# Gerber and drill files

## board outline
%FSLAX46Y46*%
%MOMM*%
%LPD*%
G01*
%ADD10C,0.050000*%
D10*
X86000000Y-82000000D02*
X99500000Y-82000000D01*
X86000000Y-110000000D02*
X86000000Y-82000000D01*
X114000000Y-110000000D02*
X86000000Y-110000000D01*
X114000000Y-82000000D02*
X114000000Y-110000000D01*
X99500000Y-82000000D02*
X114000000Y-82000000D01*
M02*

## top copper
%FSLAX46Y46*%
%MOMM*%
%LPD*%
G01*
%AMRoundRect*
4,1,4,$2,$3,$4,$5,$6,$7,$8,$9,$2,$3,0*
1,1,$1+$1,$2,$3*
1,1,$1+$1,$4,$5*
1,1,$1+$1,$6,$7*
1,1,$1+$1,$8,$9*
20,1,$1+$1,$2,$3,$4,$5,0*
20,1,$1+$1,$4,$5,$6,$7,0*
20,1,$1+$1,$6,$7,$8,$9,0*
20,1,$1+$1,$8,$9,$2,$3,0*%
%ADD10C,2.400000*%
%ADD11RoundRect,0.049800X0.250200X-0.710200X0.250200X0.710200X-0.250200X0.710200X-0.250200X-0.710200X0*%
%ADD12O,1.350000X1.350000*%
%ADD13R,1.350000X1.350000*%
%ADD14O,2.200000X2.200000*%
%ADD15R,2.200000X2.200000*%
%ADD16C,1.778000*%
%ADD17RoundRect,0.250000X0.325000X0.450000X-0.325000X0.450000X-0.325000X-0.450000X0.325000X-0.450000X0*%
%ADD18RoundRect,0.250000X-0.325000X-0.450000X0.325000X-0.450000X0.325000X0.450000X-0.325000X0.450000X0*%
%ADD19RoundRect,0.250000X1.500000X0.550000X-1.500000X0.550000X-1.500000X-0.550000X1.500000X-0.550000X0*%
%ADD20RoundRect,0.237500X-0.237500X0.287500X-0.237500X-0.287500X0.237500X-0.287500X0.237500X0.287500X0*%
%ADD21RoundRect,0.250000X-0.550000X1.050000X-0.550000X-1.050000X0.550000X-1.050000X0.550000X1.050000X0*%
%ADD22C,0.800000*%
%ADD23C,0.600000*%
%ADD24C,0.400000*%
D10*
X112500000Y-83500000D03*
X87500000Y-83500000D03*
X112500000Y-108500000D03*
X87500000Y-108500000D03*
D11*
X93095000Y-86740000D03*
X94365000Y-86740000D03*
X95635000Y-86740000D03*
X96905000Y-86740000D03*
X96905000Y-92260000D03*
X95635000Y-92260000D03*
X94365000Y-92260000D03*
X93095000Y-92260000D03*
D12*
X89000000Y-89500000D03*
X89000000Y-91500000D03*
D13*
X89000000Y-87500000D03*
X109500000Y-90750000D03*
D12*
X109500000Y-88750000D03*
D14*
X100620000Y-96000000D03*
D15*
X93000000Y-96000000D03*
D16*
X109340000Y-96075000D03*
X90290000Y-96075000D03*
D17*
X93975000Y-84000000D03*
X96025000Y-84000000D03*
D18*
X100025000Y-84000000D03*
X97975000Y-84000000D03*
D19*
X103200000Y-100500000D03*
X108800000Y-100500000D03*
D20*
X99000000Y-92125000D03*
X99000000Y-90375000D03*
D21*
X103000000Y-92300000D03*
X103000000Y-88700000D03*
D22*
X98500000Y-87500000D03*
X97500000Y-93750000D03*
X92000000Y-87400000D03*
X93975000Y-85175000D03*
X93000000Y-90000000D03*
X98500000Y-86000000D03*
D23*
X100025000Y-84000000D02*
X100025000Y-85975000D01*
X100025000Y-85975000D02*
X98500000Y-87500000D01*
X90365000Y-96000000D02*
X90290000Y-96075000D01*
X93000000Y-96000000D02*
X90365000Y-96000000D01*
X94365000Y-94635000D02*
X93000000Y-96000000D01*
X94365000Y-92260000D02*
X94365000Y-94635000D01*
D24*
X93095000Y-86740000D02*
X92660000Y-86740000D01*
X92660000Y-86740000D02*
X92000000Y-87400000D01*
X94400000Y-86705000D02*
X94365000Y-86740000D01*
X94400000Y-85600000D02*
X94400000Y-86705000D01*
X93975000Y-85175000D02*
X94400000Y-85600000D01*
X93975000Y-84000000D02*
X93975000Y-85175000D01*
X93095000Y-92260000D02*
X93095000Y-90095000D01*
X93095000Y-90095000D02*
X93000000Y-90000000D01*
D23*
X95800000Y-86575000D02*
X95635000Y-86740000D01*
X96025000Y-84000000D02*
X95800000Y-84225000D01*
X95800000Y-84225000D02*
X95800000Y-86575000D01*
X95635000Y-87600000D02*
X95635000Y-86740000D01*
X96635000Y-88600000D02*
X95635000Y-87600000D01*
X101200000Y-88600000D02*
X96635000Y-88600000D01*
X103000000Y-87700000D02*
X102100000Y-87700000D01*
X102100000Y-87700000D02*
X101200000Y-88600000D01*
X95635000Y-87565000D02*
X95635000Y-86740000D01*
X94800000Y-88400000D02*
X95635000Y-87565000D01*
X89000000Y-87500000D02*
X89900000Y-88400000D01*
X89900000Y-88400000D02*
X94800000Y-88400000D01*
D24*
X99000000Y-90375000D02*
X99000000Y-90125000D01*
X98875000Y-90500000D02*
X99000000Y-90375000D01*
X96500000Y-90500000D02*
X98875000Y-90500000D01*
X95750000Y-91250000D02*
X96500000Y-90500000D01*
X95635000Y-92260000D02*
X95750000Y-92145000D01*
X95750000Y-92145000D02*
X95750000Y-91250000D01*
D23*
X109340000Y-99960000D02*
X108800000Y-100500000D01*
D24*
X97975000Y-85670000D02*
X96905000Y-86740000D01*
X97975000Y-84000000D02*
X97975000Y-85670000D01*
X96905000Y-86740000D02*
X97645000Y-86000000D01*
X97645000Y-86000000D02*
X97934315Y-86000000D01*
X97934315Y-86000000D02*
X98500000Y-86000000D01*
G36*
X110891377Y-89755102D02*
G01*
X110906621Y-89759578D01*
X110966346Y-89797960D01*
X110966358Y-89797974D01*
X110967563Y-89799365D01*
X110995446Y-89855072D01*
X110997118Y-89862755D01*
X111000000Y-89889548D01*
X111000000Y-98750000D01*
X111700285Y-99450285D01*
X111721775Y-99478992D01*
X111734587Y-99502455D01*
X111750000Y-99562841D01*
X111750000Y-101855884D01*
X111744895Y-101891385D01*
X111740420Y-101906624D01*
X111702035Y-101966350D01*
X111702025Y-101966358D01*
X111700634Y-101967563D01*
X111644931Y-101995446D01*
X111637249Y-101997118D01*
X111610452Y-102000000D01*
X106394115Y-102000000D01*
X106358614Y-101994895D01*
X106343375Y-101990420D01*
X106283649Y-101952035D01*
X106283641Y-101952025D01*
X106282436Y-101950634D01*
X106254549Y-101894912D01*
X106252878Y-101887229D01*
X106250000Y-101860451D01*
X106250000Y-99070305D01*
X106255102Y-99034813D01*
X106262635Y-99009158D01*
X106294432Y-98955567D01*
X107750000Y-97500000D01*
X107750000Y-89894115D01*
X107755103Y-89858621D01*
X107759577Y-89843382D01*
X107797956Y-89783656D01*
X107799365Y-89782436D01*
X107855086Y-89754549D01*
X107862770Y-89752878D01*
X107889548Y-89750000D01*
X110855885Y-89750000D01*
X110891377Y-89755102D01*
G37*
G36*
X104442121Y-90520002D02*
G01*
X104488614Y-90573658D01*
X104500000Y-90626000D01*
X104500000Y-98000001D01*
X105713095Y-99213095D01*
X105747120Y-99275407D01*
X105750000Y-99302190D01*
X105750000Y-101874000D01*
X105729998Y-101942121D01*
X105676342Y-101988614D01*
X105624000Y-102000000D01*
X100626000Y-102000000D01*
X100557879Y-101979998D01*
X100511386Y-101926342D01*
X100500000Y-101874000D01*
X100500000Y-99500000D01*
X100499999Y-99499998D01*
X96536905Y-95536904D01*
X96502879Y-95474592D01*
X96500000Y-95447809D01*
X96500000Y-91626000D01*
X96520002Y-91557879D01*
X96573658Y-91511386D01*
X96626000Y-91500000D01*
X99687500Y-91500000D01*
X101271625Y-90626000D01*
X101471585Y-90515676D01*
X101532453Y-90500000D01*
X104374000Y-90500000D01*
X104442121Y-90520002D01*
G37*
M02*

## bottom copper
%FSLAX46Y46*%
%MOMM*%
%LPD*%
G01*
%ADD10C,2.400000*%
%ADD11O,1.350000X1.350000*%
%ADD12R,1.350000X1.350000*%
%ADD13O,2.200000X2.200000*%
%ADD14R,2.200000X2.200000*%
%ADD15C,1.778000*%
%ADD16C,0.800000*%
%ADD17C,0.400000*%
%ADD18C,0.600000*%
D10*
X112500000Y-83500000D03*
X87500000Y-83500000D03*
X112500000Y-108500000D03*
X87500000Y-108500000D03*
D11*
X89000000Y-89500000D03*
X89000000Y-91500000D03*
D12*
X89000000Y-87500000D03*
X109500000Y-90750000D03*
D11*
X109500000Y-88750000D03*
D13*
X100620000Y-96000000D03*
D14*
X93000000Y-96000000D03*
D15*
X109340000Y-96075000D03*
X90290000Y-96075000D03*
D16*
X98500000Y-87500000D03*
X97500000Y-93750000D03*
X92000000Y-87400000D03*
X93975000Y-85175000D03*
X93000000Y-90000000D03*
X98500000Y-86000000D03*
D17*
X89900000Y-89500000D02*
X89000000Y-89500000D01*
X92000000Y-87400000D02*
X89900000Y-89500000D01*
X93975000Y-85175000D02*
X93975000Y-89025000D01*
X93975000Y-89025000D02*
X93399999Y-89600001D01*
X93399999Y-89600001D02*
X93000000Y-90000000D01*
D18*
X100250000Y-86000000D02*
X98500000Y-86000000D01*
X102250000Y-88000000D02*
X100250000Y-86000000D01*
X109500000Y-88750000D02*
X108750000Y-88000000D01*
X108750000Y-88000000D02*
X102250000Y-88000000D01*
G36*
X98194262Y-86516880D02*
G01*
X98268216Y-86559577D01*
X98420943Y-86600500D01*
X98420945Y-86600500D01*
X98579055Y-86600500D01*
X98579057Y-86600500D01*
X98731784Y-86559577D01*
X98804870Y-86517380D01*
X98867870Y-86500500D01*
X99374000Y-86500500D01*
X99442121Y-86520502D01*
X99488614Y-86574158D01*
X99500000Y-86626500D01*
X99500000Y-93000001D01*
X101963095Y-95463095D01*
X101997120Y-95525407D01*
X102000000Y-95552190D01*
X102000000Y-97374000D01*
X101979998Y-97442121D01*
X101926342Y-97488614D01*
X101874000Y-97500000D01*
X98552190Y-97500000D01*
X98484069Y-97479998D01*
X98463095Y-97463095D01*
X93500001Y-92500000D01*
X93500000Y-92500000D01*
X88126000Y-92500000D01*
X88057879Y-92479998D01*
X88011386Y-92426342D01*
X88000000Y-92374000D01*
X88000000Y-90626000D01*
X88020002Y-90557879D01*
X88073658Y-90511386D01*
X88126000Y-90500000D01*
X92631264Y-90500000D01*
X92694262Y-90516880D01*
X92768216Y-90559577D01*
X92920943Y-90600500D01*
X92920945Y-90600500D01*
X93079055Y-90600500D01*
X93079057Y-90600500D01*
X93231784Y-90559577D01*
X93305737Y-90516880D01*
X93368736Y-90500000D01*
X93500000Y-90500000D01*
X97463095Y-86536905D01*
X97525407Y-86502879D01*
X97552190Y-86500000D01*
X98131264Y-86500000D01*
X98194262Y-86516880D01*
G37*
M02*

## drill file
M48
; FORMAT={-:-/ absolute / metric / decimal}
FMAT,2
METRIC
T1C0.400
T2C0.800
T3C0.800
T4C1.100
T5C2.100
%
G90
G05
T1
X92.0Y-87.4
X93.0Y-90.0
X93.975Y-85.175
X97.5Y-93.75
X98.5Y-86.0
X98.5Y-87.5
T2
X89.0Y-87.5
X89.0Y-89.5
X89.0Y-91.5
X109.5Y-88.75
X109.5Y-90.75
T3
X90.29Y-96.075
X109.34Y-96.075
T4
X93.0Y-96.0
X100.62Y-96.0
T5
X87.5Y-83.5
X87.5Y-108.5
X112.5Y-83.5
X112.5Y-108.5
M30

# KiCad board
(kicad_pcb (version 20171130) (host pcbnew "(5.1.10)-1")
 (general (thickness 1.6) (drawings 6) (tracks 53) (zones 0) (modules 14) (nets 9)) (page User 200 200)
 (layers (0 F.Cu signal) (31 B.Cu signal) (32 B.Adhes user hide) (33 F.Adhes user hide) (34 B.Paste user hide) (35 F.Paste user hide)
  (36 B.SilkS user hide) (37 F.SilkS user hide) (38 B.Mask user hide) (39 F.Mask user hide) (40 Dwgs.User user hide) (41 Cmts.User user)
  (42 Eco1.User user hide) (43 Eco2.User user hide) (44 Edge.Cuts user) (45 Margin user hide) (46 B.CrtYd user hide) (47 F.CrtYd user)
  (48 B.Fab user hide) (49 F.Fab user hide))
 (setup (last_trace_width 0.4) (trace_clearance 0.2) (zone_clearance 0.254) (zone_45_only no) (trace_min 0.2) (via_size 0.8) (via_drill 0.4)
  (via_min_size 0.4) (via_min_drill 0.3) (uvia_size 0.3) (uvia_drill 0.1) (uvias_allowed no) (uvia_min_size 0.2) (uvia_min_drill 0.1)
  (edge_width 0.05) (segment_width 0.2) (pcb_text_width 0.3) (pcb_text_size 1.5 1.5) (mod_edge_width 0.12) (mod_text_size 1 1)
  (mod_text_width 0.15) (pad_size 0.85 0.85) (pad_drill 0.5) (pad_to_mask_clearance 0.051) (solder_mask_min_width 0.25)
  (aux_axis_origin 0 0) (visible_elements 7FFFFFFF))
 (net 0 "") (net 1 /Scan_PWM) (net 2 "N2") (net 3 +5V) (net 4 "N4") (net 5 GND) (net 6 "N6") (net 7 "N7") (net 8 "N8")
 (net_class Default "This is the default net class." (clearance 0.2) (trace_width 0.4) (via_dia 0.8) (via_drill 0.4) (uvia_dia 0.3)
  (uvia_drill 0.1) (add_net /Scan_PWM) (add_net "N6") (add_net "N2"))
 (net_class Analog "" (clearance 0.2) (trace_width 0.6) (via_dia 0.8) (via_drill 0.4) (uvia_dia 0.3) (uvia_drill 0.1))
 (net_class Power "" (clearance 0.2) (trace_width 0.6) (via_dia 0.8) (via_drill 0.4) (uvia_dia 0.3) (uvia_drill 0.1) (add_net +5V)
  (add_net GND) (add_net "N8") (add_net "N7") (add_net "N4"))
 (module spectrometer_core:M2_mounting (layer F.Cu) (at 112.5 83.5)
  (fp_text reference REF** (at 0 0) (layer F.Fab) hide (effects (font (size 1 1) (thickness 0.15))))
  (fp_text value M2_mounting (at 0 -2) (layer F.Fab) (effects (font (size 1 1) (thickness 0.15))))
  (pad "" np_thru_hole circle (at 0 0) (size 2.4 2.4) (drill 2.1) (layers *.Cu *.Mask) (zone_connect 0)))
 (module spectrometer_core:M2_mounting (layer F.Cu) (at 87.5 83.5)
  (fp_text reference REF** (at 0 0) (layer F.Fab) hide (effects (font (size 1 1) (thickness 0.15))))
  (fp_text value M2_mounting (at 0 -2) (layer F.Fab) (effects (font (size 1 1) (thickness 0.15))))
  (pad "" np_thru_hole circle (at 0 0) (size 2.4 2.4) (drill 2.1) (layers *.Cu *.Mask) (zone_connect 0)))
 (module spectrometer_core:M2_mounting (layer F.Cu) (at 112.5 108.5)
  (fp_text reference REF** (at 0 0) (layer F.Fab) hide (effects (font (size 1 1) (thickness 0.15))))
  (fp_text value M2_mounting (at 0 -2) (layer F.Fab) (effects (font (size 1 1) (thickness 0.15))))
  (pad "" np_thru_hole circle (at 0 0) (size 2.4 2.4) (drill 2.1) (layers *.Cu *.Mask) (zone_connect 0)))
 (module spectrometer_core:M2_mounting (layer F.Cu) (at 87.5 108.5)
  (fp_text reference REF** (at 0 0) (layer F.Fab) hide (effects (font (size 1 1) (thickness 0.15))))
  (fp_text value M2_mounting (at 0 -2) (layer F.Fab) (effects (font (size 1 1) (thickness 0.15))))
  (pad "" np_thru_hole circle (at 0 0) (size 2.4 2.4) (drill 2.1) (layers *.Cu *.Mask) (zone_connect 0)))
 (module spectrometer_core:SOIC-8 (layer F.Cu) (at 95 89.5 90)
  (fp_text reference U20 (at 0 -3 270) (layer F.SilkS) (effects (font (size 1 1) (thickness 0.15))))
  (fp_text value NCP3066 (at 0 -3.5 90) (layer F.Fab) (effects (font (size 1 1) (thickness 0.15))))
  (pad 8 smd roundrect (at 2.76 -1.905 90) (size 1.52 0.6) (layers F.Cu F.Paste F.Mask) (roundrect_rratio 0.083) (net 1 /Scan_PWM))
  (pad 7 smd roundrect (at 2.76 -0.635 90) (size 1.52 0.6) (layers F.Cu F.Paste F.Mask) (roundrect_rratio 0.083) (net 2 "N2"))
  (pad 6 smd roundrect (at 2.76 0.635 90) (size 1.52 0.6) (layers F.Cu F.Paste F.Mask) (roundrect_rratio 0.083) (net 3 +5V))
  (pad 5 smd roundrect (at 2.76 1.905 90) (size 1.52 0.6) (layers F.Cu F.Paste F.Mask) (roundrect_rratio 0.083) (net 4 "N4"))
  (pad 4 smd roundrect (at -2.76 1.905 90) (size 1.52 0.6) (layers F.Cu F.Paste F.Mask) (roundrect_rratio 0.083) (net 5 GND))
  (pad 3 smd roundrect (at -2.76 0.635 90) (size 1.52 0.6) (layers F.Cu F.Paste F.Mask) (roundrect_rratio 0.083) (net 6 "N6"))
  (pad 2 smd roundrect (at -2.76 -0.635 90) (size 1.52 0.6) (layers F.Cu F.Paste F.Mask) (roundrect_rratio 0.083) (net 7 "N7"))
  (pad 1 smd roundrect (at -2.76 -1.905 90) (size 1.52 0.6) (layers F.Cu F.Paste F.Mask) (roundrect_rratio 0.083) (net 2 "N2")))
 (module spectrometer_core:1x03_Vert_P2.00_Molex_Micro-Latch (layer F.Cu) (at 89 89.5 180)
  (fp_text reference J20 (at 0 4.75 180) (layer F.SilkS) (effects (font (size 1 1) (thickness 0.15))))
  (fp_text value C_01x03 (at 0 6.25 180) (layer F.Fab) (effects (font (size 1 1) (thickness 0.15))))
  (pad 2 thru_hole oval (at 0 0 180) (size 1.35 1.35) (drill 0.8) (layers *.Cu *.Mask) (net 1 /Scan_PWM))
  (pad 3 thru_hole oval (at 0 -2 180) (size 1.35 1.35) (drill 0.8) (layers *.Cu *.Mask) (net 5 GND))
  (pad 1 thru_hole rect (at 0 2 180) (size 1.35 1.35) (drill 0.8) (layers *.Cu *.Mask) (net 3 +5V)))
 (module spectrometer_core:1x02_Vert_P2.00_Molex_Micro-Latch (layer F.Cu) (at 109.5 89.75)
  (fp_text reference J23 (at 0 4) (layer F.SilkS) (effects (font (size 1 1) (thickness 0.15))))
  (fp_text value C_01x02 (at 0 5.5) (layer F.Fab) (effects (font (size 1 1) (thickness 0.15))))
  (pad 1 thru_hole rect (at 0 1) (size 1.35 1.35) (drill 0.8) (layers *.Cu *.Mask) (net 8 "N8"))
  (pad 2 thru_hole oval (at 0 -1) (size 1.35 1.35) (drill 0.8) (layers *.Cu *.Mask) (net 4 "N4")))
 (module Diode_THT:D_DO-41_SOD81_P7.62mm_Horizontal (layer F.Cu) (at 93 96)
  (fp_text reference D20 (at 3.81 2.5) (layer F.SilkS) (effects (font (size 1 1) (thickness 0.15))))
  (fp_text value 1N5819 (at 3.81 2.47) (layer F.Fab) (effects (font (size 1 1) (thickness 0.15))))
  (pad 2 thru_hole oval (at 7.62 0) (size 2.2 2.2) (drill 1.1) (layers *.Cu *.Mask) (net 5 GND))
  (pad 1 thru_hole rect (at 0 0) (size 2.2 2.2) (drill 1.1) (layers *.Cu *.Mask) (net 7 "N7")))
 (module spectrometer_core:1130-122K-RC (layer F.Cu) (at 99.815 96.075)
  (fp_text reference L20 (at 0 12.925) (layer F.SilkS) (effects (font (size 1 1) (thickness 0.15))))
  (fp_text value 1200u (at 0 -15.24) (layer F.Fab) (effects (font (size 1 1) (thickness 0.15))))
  (pad 2 thru_hole circle (at 9.525 0) (size 1.778 1.778) (drill 0.8001) (layers *.Cu *.Mask) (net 8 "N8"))
  (pad 1 thru_hole circle (at -9.525 0) (size 1.778 1.778) (drill 0.8001) (layers *.Cu *.Mask) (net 7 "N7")))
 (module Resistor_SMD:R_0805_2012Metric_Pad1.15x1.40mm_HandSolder (layer F.Cu) (at 95 84 180)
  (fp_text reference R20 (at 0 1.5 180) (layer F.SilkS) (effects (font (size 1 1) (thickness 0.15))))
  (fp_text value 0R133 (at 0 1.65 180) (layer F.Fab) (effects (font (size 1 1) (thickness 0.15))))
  (pad 2 smd roundrect (at 1.025 0 180) (size 1.15 1.4) (layers F.Cu F.Paste F.Mask) (roundrect_rratio 0.217391) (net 2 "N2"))
  (pad 1 smd roundrect (at -1.025 0 180) (size 1.15 1.4) (layers F.Cu F.Paste F.Mask) (roundrect_rratio 0.217391) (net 3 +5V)))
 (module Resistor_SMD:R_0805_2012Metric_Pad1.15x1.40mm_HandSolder (layer F.Cu) (at 99 84)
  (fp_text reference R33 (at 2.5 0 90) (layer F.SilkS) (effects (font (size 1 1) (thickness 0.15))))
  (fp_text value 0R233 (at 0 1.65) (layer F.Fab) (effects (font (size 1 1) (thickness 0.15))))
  (pad 2 smd roundrect (at 1.025 0) (size 1.15 1.4) (layers F.Cu F.Paste F.Mask) (roundrect_rratio 0.217391) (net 5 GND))
  (pad 1 smd roundrect (at -1.025 0) (size 1.15 1.4) (layers F.Cu F.Paste F.Mask) (roundrect_rratio 0.217391) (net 4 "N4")))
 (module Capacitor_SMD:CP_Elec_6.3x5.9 (layer F.Cu) (at 106 100.5 180)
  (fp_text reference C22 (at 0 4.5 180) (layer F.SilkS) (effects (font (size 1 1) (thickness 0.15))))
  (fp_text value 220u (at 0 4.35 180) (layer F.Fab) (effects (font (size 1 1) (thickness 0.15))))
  (pad 2 smd roundrect (at 2.8 0 180) (size 3.5 1.6) (layers F.Cu F.Paste F.Mask) (roundrect_rratio 0.15625) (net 5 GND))
  (pad 1 smd roundrect (at -2.8 0 180) (size 3.5 1.6) (layers F.Cu F.Paste F.Mask) (roundrect_rratio 0.15625) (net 8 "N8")))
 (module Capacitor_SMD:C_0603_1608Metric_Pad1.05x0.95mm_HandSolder (layer F.Cu) (at 99 91.25 270)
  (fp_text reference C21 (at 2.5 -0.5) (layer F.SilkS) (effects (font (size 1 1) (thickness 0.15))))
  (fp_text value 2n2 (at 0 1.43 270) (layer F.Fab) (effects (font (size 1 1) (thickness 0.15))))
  (pad 2 smd roundrect (at 0.875 0 270) (size 1.05 0.95) (layers F.Cu F.Paste F.Mask) (roundrect_rratio 0.25) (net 5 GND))
  (pad 1 smd roundrect (at -0.875 0 270) (size 1.05 0.95) (layers F.Cu F.Paste F.Mask) (roundrect_rratio 0.25) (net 6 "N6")))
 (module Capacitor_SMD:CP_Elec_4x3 (layer F.Cu) (at 103 90.5 270)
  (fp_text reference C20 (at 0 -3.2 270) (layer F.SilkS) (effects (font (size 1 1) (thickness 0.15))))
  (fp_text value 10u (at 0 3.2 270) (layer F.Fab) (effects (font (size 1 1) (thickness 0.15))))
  (pad 2 smd roundrect (at 1.8 0 270) (size 2.6 1.6) (layers F.Cu F.Paste F.Mask) (roundrect_rratio 0.15625) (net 5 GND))
  (pad 1 smd roundrect (at -1.8 0 270) (size 2.6 1.6) (layers F.Cu F.Paste F.Mask) (roundrect_rratio 0.15625) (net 3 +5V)))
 (gr_line (start 86 82) (end 99.5 82) (layer Edge.Cuts) (width 0.05))
 (gr_line (start 86 110) (end 86 82) (layer Edge.Cuts) (width 0.05))
 (gr_line (start 114 110) (end 86 110) (layer Edge.Cuts) (width 0.05))
 (gr_line (start 114 82) (end 114 110) (layer Edge.Cuts) (width 0.05))
 (gr_line (start 99.5 82) (end 114 82) (layer Edge.Cuts) (width 0.05))
 (via (at 98.5 87.5) (size 0.8) (drill 0.4) (layers F.Cu B.Cu) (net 5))
 (segment (start 100.025 84) (end 100.025 85.975) (width 0.6) (layer F.Cu) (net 5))
 (segment (start 100.025 85.975) (end 98.5 87.5) (width 0.6) (layer F.Cu) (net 5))
 (via (at 97.5 93.75) (size 0.8) (drill 0.4) (layers F.Cu B.Cu) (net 5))
 (segment (start 90.365 96) (end 90.29 96.075) (width 0.6) (layer F.Cu) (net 7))
 (segment (start 93 96) (end 90.365 96) (width 0.6) (layer F.Cu) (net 7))
 (segment (start 94.365 94.635) (end 93 96) (width 0.6) (layer F.Cu) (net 7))
 (segment (start 94.365 92.26) (end 94.365 94.635) (width 0.6) (layer F.Cu) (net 7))
 (via (at 92 87.4) (size 0.8) (drill 0.4) (layers F.Cu B.Cu) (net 1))
 (segment (start 93.095 86.74) (end 92.66 86.74) (width 0.4) (layer F.Cu) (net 1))
 (segment (start 92.66 86.74) (end 92 87.4) (width 0.4) (layer F.Cu) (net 1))
 (segment (start 89.9 89.5) (end 89 89.5) (width 0.4) (layer B.Cu) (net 1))
 (segment (start 92 87.4) (end 89.9 89.5) (width 0.4) (layer B.Cu) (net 1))
 (segment (start 94.4 86.705) (end 94.365 86.74) (width 0.4) (layer F.Cu) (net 2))
 (segment (start 94.4 85.6) (end 94.4 86.705) (width 0.4) (layer F.Cu) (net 2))
 (segment (start 93.975 85.175) (end 94.4 85.6) (width 0.4) (layer F.Cu) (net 2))
 (via (at 93.975 85.175) (size 0.8) (drill 0.4) (layers F.Cu B.Cu) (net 2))
 (segment (start 93.975 84) (end 93.975 85.175) (width 0.4) (layer F.Cu) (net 2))
 (via (at 93 90) (size 0.8) (drill 0.4) (layers F.Cu B.Cu) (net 2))
 (segment (start 93.095 92.26) (end 93.095 90.095) (width 0.4) (layer F.Cu) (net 2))
 (segment (start 93.095 90.095) (end 93 90) (width 0.4) (layer F.Cu) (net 2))
 (segment (start 93.975 85.175) (end 93.975 89.025) (width 0.4) (layer B.Cu) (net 2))
 (segment (start 93.975 89.025) (end 93.399999 89.600001) (width 0.4) (layer B.Cu) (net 2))
 (segment (start 93.399999 89.600001) (end 93 90) (width 0.4) (layer B.Cu) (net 2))
 (segment (start 95.8 86.575) (end 95.635 86.74) (width 0.6) (layer F.Cu) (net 3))
 (segment (start 96.025 84) (end 95.8 84.225) (width 0.6) (layer F.Cu) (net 3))
 (segment (start 95.8 84.225) (end 95.8 86.575) (width 0.6) (layer F.Cu) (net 3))
 (segment (start 95.635 87.6) (end 95.635 86.74) (width 0.6) (layer F.Cu) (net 3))
 (segment (start 96.635 88.6) (end 95.635 87.6) (width 0.6) (layer F.Cu) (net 3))
 (segment (start 101.2 88.6) (end 96.635 88.6) (width 0.6) (layer F.Cu) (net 3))
 (segment (start 103 87.7) (end 102.1 87.7) (width 0.6) (layer F.Cu) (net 3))
 (segment (start 102.1 87.7) (end 101.2 88.6) (width 0.6) (layer F.Cu) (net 3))
 (segment (start 95.635 87.565) (end 95.635 86.74) (width 0.6) (layer F.Cu) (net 3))
 (segment (start 94.8 88.4) (end 95.635 87.565) (width 0.6) (layer F.Cu) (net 3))
 (segment (start 89 87.5) (end 89.9 88.4) (width 0.6) (layer F.Cu) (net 3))
 (segment (start 89.9 88.4) (end 94.8 88.4) (width 0.6) (layer F.Cu) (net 3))
 (segment (start 99 90.375) (end 99 90.125) (width 0.4) (layer F.Cu) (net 6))
 (segment (start 98.875 90.5) (end 99 90.375) (width 0.4) (layer F.Cu) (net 6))
 (segment (start 96.5 90.5) (end 98.875 90.5) (width 0.4) (layer F.Cu) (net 6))
 (segment (start 95.75 91.25) (end 96.5 90.5) (width 0.4) (layer F.Cu) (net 6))
 (segment (start 95.635 92.26) (end 95.75 92.145) (width 0.4) (layer F.Cu) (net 6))
 (segment (start 95.75 92.145) (end 95.75 91.25) (width 0.4) (layer F.Cu) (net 6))
 (segment (start 109.34 99.96) (end 108.8 100.5) (width 0.6) (layer F.Cu) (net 8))
 (segment (start 97.975 85.67) (end 96.905 86.74) (width 0.4) (layer F.Cu) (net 4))
 (segment (start 97.975 84) (end 97.975 85.67) (width 0.4) (layer F.Cu) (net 4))
 (via (at 98.5 86) (size 0.8) (drill 0.4) (layers F.Cu B.Cu) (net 4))
 (segment (start 96.905 86.74) (end 97.645 86) (width 0.4) (layer F.Cu) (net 4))
 (segment (start 97.645 86) (end 97.934315 86) (width 0.4) (layer F.Cu) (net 4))
 (segment (start 97.934315 86) (end 98.5 86) (width 0.4) (layer F.Cu) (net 4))
 (segment (start 100.25 86) (end 98.5 86) (width 0.6) (layer B.Cu) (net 4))
 (segment (start 102.25 88) (end 100.25 86) (width 0.6) (layer B.Cu) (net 4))
 (segment (start 109.5 88.75) (end 108.75 88) (width 0.6) (layer B.Cu) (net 4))
 (segment (start 108.75 88) (end 102.25 88) (width 0.6) (layer B.Cu) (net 4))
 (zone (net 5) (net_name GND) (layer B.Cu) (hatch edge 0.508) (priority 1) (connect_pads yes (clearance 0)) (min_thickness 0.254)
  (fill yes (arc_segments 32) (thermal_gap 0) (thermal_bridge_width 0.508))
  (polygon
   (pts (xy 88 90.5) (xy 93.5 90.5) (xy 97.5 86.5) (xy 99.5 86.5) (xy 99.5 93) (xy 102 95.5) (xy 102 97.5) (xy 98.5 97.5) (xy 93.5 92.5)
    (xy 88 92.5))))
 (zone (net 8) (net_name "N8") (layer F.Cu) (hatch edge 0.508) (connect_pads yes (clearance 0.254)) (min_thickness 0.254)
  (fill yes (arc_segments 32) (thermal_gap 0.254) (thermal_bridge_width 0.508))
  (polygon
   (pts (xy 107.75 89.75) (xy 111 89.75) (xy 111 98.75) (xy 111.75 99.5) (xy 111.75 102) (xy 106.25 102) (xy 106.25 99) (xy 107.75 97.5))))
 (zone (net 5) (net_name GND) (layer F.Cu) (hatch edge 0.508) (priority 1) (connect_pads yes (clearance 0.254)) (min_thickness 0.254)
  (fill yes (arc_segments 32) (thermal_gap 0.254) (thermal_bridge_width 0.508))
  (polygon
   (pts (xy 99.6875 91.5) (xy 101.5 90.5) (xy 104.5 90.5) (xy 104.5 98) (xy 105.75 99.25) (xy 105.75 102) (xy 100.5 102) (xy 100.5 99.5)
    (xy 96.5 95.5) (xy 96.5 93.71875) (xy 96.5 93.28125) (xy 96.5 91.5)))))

